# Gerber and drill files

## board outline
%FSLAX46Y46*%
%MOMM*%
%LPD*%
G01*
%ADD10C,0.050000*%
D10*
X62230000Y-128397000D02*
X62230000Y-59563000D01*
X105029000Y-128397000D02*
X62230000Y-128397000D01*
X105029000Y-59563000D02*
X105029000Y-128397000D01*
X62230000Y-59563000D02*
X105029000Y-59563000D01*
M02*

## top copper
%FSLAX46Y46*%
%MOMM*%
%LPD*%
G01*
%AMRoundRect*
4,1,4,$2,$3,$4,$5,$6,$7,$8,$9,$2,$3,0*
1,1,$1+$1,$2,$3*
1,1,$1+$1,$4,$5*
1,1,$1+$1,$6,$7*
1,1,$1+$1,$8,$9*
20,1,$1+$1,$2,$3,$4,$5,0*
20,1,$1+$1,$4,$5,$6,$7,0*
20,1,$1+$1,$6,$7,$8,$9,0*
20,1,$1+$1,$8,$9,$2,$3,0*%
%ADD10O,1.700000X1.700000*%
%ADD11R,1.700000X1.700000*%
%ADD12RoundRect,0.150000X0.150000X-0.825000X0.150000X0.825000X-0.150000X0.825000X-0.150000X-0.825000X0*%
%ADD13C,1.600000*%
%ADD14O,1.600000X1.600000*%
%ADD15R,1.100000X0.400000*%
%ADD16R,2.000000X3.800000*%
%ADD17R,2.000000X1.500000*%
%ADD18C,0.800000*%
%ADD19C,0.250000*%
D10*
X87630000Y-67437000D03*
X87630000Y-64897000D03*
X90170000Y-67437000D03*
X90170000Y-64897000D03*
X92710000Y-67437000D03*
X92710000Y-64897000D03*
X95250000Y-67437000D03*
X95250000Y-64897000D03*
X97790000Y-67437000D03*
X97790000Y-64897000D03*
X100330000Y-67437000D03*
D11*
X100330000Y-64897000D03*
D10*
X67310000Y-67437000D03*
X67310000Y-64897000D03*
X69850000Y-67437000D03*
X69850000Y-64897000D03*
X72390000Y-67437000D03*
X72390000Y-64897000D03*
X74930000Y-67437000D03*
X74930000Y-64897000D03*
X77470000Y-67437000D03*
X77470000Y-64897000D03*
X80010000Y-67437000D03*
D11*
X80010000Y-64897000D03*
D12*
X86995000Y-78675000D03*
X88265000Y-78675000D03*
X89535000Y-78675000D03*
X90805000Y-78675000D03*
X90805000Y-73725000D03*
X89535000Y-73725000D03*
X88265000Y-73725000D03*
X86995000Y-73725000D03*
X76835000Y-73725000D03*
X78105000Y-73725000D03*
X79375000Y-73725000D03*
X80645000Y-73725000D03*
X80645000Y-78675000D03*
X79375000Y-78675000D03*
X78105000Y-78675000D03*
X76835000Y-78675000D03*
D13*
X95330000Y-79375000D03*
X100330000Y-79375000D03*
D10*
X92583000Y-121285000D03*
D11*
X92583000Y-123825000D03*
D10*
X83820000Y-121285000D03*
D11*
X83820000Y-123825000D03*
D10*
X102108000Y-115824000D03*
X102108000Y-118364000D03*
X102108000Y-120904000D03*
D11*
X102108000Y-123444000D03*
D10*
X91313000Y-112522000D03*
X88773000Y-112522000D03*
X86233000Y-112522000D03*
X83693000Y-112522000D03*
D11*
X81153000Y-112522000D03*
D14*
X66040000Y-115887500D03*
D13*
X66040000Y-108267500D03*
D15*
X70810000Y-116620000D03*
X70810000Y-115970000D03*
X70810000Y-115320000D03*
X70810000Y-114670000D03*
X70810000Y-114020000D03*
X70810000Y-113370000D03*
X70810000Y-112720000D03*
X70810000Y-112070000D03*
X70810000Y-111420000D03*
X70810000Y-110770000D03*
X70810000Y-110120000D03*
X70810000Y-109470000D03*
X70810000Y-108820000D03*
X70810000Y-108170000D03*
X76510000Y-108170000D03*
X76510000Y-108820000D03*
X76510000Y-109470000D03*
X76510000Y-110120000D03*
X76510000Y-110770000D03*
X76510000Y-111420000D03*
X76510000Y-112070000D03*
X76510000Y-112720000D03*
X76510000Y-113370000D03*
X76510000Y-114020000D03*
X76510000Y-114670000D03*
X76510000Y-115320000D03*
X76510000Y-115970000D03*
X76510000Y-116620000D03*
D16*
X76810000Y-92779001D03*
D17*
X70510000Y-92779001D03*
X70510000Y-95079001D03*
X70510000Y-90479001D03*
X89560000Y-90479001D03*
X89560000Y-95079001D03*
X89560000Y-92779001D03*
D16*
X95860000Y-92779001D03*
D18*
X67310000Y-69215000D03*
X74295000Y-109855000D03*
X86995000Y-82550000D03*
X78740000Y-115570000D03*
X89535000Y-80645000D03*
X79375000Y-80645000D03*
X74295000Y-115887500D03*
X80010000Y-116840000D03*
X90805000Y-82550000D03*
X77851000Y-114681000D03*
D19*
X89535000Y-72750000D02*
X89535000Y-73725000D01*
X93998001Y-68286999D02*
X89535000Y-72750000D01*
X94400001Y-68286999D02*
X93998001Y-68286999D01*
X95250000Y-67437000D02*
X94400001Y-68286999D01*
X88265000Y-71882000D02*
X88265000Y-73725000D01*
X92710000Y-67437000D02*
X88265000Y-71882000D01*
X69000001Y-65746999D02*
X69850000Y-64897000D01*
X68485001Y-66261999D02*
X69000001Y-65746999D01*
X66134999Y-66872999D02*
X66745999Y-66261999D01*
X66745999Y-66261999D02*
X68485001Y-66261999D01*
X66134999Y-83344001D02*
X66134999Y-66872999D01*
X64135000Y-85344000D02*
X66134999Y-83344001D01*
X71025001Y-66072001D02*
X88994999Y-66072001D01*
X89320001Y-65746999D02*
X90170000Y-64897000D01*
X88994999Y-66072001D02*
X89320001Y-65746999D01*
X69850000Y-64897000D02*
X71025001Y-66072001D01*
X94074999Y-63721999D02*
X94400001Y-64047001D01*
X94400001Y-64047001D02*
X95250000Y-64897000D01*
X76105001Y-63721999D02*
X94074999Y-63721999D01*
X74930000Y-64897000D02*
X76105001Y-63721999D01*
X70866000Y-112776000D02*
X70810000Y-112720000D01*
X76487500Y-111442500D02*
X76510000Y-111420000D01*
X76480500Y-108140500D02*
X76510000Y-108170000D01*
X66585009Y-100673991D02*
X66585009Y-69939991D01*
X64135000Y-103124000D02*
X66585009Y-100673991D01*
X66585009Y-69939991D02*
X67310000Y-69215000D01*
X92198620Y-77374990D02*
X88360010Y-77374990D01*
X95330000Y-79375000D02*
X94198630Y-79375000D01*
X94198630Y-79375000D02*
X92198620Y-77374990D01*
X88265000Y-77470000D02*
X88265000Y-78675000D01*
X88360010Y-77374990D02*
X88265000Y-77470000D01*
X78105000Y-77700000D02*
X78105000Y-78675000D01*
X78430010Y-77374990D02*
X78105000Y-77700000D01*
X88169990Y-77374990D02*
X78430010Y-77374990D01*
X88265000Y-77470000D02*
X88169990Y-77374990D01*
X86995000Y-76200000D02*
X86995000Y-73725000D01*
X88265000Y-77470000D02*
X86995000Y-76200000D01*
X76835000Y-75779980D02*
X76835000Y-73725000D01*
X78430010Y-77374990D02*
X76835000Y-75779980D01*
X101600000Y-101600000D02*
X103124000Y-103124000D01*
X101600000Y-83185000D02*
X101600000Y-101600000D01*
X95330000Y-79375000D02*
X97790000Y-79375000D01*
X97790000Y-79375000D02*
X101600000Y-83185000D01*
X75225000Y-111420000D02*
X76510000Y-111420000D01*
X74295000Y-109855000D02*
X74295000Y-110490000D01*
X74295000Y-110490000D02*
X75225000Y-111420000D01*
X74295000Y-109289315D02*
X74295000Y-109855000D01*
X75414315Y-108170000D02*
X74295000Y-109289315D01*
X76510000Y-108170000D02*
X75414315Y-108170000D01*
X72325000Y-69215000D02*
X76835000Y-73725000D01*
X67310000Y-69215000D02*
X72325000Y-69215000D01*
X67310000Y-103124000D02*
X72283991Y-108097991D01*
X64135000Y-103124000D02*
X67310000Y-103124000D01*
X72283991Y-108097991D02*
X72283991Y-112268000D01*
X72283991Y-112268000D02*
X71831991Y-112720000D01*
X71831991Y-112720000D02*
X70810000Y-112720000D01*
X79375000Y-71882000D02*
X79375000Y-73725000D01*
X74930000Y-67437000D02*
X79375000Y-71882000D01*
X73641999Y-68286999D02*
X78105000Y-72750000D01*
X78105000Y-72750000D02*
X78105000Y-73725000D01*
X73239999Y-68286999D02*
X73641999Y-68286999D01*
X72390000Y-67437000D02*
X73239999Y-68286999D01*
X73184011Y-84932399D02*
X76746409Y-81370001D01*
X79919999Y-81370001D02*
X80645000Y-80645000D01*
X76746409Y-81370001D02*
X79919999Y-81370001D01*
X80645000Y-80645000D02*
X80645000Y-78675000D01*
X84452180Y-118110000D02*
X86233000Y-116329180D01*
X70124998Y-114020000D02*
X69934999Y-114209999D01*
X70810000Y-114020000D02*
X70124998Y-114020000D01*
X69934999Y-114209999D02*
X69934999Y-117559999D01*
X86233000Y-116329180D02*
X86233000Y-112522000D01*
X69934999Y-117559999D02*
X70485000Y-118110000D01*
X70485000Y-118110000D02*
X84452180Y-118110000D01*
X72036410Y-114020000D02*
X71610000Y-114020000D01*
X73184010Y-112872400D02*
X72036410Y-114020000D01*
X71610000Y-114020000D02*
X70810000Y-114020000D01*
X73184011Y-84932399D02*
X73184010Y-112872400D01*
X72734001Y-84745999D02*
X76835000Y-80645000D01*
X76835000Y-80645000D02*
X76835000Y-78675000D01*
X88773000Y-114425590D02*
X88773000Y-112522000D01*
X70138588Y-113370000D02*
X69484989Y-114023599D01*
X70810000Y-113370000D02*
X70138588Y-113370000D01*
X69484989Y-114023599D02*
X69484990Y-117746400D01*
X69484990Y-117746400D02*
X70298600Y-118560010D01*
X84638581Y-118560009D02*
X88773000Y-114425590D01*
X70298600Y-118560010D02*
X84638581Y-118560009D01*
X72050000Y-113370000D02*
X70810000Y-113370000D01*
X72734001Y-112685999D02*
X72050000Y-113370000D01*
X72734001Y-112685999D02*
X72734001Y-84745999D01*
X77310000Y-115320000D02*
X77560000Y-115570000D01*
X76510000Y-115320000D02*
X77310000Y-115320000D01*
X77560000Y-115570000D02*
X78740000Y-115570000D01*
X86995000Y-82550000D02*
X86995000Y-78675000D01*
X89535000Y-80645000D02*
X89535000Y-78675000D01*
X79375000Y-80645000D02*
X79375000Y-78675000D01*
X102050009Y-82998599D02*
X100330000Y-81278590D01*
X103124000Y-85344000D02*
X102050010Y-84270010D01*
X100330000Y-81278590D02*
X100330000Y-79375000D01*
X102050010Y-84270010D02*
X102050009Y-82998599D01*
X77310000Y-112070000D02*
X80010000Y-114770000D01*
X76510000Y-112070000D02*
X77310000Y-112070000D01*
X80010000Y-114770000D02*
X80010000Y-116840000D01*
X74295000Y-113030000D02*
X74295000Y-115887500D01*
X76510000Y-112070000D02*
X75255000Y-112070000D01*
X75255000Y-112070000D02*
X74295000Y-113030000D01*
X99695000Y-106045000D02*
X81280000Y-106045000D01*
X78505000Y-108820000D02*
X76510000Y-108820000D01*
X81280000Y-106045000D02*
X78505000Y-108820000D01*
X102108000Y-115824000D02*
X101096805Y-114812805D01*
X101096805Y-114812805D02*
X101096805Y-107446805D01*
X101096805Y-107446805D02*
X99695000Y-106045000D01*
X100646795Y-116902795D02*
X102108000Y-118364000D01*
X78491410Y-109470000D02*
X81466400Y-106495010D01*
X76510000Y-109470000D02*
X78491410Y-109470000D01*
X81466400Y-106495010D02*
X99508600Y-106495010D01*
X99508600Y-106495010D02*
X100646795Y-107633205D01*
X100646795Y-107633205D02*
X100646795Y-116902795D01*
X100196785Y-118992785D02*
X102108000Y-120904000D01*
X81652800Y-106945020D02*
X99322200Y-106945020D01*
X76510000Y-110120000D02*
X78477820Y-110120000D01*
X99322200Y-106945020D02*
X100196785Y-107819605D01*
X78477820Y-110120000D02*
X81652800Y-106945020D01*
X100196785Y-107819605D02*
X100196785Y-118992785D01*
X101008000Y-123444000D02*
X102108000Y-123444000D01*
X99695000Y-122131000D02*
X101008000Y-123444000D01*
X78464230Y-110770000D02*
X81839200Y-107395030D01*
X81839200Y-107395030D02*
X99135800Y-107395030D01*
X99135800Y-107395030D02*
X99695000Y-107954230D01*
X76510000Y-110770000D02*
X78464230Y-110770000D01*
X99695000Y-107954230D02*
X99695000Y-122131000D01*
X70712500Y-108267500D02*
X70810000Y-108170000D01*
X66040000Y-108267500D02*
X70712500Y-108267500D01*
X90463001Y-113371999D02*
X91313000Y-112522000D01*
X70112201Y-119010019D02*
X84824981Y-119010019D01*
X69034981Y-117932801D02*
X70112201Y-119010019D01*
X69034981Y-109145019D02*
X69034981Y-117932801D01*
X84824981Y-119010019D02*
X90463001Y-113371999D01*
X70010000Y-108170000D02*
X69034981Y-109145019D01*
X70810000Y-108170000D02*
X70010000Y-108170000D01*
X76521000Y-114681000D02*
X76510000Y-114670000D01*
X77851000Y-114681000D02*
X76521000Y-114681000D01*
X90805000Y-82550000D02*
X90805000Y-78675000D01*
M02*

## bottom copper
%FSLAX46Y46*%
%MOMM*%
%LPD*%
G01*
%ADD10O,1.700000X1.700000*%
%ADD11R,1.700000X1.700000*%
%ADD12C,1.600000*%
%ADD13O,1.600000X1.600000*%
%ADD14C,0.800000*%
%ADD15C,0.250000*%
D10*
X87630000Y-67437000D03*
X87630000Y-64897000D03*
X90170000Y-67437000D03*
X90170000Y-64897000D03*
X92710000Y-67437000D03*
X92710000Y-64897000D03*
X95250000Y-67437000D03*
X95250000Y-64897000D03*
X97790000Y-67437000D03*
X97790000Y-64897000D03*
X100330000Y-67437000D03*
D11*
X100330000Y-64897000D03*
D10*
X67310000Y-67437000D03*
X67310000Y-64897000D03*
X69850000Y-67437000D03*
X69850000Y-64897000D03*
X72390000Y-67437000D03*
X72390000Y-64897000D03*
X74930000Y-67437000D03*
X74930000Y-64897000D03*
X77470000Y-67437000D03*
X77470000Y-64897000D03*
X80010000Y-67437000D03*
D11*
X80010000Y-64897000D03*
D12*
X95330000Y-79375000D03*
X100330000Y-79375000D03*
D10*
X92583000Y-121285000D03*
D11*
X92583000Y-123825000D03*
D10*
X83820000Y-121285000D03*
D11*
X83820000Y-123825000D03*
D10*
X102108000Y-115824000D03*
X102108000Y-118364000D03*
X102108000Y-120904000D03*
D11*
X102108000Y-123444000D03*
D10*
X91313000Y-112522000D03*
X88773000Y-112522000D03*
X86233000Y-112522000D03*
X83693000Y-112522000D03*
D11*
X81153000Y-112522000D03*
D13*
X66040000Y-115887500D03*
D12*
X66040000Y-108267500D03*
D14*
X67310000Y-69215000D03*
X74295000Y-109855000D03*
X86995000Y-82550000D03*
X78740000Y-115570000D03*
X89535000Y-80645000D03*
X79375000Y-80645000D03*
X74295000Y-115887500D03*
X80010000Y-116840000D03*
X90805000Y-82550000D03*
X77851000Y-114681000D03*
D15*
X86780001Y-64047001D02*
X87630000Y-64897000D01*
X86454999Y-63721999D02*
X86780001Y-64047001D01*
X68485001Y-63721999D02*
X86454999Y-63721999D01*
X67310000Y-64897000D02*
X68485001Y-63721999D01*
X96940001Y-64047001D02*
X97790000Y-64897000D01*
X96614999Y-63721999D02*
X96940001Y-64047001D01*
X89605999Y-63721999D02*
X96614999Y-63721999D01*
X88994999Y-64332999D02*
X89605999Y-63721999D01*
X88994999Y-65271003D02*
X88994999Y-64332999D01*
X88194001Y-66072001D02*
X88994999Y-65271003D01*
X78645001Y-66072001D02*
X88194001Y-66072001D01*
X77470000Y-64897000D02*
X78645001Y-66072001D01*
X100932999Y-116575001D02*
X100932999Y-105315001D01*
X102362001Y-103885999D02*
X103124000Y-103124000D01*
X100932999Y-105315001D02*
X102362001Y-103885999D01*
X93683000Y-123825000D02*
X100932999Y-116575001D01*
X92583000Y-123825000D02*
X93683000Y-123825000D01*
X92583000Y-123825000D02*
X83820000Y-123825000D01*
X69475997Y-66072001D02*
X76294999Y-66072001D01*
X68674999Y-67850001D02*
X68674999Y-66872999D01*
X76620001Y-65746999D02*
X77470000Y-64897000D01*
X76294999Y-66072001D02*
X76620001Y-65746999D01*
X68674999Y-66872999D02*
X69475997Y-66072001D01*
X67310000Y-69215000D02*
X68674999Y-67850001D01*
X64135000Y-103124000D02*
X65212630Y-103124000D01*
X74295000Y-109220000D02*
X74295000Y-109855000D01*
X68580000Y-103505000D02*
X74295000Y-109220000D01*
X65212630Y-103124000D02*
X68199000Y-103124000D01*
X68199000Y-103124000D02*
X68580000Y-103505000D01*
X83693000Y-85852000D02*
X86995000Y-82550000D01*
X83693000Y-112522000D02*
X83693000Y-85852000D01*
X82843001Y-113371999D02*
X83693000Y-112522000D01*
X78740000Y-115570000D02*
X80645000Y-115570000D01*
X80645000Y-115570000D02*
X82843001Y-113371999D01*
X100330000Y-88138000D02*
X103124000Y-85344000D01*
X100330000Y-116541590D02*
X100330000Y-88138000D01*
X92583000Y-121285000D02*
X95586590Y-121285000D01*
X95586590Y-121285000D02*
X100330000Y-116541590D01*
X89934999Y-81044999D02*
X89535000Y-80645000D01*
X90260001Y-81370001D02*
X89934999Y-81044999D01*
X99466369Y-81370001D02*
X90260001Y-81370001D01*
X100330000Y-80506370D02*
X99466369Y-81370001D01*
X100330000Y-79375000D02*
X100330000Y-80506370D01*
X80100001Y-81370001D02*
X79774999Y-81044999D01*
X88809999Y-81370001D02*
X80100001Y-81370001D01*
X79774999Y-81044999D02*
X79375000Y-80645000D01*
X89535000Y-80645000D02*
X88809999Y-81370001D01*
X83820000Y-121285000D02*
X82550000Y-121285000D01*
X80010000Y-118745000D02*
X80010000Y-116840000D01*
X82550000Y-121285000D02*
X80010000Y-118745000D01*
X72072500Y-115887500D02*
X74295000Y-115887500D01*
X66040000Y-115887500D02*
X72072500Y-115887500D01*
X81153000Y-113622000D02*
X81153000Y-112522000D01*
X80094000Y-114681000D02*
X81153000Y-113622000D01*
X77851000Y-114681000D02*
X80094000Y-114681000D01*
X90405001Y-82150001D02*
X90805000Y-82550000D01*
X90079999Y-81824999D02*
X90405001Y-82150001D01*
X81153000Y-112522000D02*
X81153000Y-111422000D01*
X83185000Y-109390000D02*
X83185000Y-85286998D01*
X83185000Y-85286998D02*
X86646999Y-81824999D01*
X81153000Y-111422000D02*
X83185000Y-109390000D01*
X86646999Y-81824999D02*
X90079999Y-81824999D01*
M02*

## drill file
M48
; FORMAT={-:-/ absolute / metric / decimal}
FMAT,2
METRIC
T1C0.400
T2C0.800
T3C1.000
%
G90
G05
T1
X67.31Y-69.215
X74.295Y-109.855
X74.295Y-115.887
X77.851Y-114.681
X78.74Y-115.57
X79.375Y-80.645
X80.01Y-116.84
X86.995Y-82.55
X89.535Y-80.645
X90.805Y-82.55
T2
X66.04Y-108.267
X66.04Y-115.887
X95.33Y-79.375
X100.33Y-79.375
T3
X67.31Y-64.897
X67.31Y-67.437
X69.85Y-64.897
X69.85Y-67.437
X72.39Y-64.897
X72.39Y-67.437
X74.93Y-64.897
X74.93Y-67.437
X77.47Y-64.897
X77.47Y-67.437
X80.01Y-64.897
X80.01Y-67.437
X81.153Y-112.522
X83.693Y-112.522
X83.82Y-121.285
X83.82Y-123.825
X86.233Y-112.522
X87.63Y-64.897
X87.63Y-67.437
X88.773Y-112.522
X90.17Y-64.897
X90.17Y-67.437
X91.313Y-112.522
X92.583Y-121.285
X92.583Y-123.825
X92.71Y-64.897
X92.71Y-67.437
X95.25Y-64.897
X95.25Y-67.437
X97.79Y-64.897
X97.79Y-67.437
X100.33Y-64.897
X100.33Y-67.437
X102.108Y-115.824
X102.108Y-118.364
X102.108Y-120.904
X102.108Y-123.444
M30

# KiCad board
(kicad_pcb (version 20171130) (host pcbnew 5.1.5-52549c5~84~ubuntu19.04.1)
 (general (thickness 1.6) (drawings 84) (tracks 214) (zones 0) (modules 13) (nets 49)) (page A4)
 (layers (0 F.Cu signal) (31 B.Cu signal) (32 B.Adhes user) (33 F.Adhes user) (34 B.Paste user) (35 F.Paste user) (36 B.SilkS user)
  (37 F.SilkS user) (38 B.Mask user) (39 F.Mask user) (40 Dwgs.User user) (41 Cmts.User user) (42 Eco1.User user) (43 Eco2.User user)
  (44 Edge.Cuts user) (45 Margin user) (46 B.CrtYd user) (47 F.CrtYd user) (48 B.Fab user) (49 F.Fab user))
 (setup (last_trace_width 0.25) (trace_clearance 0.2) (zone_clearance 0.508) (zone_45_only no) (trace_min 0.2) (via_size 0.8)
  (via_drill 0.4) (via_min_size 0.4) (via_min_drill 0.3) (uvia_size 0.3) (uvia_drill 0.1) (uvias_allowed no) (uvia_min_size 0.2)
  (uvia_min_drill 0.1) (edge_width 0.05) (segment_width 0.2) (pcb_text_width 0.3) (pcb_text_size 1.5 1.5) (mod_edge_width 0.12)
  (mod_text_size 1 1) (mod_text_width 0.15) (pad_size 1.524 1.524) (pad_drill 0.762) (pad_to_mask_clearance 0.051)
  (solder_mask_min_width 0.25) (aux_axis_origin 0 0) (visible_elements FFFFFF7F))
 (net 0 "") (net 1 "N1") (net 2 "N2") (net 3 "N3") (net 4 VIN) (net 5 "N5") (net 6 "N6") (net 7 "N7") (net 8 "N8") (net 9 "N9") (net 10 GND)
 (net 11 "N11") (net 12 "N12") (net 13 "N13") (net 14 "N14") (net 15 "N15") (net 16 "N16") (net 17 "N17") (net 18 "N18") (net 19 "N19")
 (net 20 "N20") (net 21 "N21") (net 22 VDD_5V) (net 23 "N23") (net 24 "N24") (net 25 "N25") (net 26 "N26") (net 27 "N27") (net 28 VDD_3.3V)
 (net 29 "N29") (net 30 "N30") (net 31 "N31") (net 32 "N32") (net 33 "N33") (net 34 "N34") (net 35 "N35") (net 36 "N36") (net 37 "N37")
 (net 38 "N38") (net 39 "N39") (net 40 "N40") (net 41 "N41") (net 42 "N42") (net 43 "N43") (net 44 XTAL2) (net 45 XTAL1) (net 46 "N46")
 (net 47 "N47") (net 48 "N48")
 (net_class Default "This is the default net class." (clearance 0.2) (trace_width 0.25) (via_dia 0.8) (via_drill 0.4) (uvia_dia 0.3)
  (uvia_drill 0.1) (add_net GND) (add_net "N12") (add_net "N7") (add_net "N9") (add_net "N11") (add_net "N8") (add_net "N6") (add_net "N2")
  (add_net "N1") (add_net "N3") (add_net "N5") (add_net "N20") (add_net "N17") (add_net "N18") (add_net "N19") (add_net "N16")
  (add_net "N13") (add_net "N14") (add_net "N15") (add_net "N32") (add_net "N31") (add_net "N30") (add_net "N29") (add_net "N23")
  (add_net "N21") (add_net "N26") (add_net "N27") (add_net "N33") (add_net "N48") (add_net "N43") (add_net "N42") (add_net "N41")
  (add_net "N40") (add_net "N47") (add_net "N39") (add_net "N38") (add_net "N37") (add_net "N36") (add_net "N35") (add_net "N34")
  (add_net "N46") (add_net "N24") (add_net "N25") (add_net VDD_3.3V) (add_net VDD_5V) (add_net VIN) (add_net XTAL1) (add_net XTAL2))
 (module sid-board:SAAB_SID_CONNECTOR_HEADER (layer F.Cu) (at 93.98 66.04)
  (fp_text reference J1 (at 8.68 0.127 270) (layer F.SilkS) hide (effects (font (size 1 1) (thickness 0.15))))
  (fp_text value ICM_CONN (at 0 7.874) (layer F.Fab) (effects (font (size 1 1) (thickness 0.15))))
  (pad 7 thru_hole oval (at -6.35 1.397 270) (size 1.7 1.7) (drill 1) (layers *.Cu *.Mask) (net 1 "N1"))
  (pad 6 thru_hole oval (at -6.35 -1.143 270) (size 1.7 1.7) (drill 1) (layers *.Cu *.Mask) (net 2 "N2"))
  (pad 8 thru_hole oval (at -3.81 1.397 270) (size 1.7 1.7) (drill 1) (layers *.Cu *.Mask) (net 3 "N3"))
  (pad 5 thru_hole oval (at -3.81 -1.143 270) (size 1.7 1.7) (drill 1) (layers *.Cu *.Mask) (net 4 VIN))
  (pad 9 thru_hole oval (at -1.27 1.397 270) (size 1.7 1.7) (drill 1) (layers *.Cu *.Mask) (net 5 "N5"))
  (pad 4 thru_hole oval (at -1.27 -1.143 270) (size 1.7 1.7) (drill 1) (layers *.Cu *.Mask) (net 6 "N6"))
  (pad 10 thru_hole oval (at 1.27 1.397 270) (size 1.7 1.7) (drill 1) (layers *.Cu *.Mask) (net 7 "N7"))
  (pad 3 thru_hole oval (at 1.27 -1.143 270) (size 1.7 1.7) (drill 1) (layers *.Cu *.Mask) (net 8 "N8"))
  (pad 11 thru_hole oval (at 3.81 1.397 270) (size 1.7 1.7) (drill 1) (layers *.Cu *.Mask) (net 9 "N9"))
  (pad 2 thru_hole oval (at 3.81 -1.143 270) (size 1.7 1.7) (drill 1) (layers *.Cu *.Mask) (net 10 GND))
  (pad 12 thru_hole oval (at 6.35 1.397 270) (size 1.7 1.7) (drill 1) (layers *.Cu *.Mask) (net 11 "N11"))
  (pad 1 thru_hole rect (at 6.35 -1.143 270) (size 1.7 1.7) (drill 1) (layers *.Cu *.Mask) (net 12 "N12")))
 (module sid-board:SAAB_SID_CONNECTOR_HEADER (layer F.Cu) (at 73.66 66.04)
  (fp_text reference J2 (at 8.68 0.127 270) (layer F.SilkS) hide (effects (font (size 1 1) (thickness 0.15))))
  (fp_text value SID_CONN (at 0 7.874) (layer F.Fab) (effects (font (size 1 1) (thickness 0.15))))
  (pad 7 thru_hole oval (at -6.35 1.397 270) (size 1.7 1.7) (drill 1) (layers *.Cu *.Mask) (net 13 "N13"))
  (pad 6 thru_hole oval (at -6.35 -1.143 270) (size 1.7 1.7) (drill 1) (layers *.Cu *.Mask) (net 2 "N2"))
  (pad 8 thru_hole oval (at -3.81 1.397 270) (size 1.7 1.7) (drill 1) (layers *.Cu *.Mask) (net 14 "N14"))
  (pad 5 thru_hole oval (at -3.81 -1.143 270) (size 1.7 1.7) (drill 1) (layers *.Cu *.Mask) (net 4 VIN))
  (pad 9 thru_hole oval (at -1.27 1.397 270) (size 1.7 1.7) (drill 1) (layers *.Cu *.Mask) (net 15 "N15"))
  (pad 4 thru_hole oval (at -1.27 -1.143 270) (size 1.7 1.7) (drill 1) (layers *.Cu *.Mask) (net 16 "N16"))
  (pad 10 thru_hole oval (at 1.27 1.397 270) (size 1.7 1.7) (drill 1) (layers *.Cu *.Mask) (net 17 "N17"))
  (pad 3 thru_hole oval (at 1.27 -1.143 270) (size 1.7 1.7) (drill 1) (layers *.Cu *.Mask) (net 8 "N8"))
  (pad 11 thru_hole oval (at 3.81 1.397 270) (size 1.7 1.7) (drill 1) (layers *.Cu *.Mask) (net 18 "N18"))
  (pad 2 thru_hole oval (at 3.81 -1.143 270) (size 1.7 1.7) (drill 1) (layers *.Cu *.Mask) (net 10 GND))
  (pad 12 thru_hole oval (at 6.35 1.397 270) (size 1.7 1.7) (drill 1) (layers *.Cu *.Mask) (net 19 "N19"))
  (pad 1 thru_hole rect (at 6.35 -1.143 270) (size 1.7 1.7) (drill 1) (layers *.Cu *.Mask) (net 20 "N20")))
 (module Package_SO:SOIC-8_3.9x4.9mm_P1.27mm (layer F.Cu) (at 88.9 76.2 90)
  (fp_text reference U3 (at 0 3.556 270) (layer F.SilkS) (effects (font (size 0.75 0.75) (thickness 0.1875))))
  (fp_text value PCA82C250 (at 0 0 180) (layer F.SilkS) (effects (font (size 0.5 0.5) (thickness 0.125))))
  (pad 1 smd roundrect (at -2.475 -1.905 90) (size 1.95 0.6) (layers F.Cu F.Paste F.Mask) (roundrect_rratio 0.25) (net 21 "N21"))
  (pad 2 smd roundrect (at -2.475 -0.635 90) (size 1.95 0.6) (layers F.Cu F.Paste F.Mask) (roundrect_rratio 0.25) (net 10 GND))
  (pad 3 smd roundrect (at -2.475 0.635 90) (size 1.95 0.6) (layers F.Cu F.Paste F.Mask) (roundrect_rratio 0.25) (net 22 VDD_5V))
  (pad 4 smd roundrect (at -2.475 1.905 90) (size 1.95 0.6) (layers F.Cu F.Paste F.Mask) (roundrect_rratio 0.25) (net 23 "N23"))
  (pad 5 smd roundrect (at 2.475 1.905 90) (size 1.95 0.6) (layers F.Cu F.Paste F.Mask) (roundrect_rratio 0.25) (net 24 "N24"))
  (pad 6 smd roundrect (at 2.475 0.635 90) (size 1.95 0.6) (layers F.Cu F.Paste F.Mask) (roundrect_rratio 0.25) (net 7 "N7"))
  (pad 7 smd roundrect (at 2.475 -0.635 90) (size 1.95 0.6) (layers F.Cu F.Paste F.Mask) (roundrect_rratio 0.25) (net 5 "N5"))
  (pad 8 smd roundrect (at 2.475 -1.905 90) (size 1.95 0.6) (layers F.Cu F.Paste F.Mask) (roundrect_rratio 0.25) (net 10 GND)))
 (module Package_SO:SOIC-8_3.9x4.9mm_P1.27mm (layer F.Cu) (at 78.74 76.2 90)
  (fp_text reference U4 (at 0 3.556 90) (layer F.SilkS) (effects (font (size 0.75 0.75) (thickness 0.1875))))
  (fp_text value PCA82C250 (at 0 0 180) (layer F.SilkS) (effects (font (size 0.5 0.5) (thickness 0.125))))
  (pad 8 smd roundrect (at 2.475 -1.905 90) (size 1.95 0.6) (layers F.Cu F.Paste F.Mask) (roundrect_rratio 0.25) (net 10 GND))
  (pad 7 smd roundrect (at 2.475 -0.635 90) (size 1.95 0.6) (layers F.Cu F.Paste F.Mask) (roundrect_rratio 0.25) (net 15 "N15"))
  (pad 6 smd roundrect (at 2.475 0.635 90) (size 1.95 0.6) (layers F.Cu F.Paste F.Mask) (roundrect_rratio 0.25) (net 17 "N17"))
  (pad 5 smd roundrect (at 2.475 1.905 90) (size 1.95 0.6) (layers F.Cu F.Paste F.Mask) (roundrect_rratio 0.25) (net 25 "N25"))
  (pad 4 smd roundrect (at -2.475 1.905 90) (size 1.95 0.6) (layers F.Cu F.Paste F.Mask) (roundrect_rratio 0.25) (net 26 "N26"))
  (pad 3 smd roundrect (at -2.475 0.635 90) (size 1.95 0.6) (layers F.Cu F.Paste F.Mask) (roundrect_rratio 0.25) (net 22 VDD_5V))
  (pad 2 smd roundrect (at -2.475 -0.635 90) (size 1.95 0.6) (layers F.Cu F.Paste F.Mask) (roundrect_rratio 0.25) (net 10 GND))
  (pad 1 smd roundrect (at -2.475 -1.905 90) (size 1.95 0.6) (layers F.Cu F.Paste F.Mask) (roundrect_rratio 0.25) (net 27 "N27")))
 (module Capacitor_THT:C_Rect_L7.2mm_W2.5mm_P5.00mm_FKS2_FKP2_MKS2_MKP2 (layer F.Cu) (at 100.33 79.375 180)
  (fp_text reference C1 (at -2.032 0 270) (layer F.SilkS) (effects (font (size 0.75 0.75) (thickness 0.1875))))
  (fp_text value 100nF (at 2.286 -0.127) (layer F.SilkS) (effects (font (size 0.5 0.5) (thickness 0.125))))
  (pad 2 thru_hole circle (at 5 0 180) (size 1.6 1.6) (drill 0.8) (layers *.Cu *.Mask) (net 10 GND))
  (pad 1 thru_hole circle (at 0 0 180) (size 1.6 1.6) (drill 0.8) (layers *.Cu *.Mask) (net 22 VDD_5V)))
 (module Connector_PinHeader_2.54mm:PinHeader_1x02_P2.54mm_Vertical (layer F.Cu) (at 92.583 123.825 180)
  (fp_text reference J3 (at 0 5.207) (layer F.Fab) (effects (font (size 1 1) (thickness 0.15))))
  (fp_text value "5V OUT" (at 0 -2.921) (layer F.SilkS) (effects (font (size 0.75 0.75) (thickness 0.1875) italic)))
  (pad 2 thru_hole oval (at 0 2.54 180) (size 1.7 1.7) (drill 1) (layers *.Cu *.Mask) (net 22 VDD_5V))
  (pad 1 thru_hole rect (at 0 0 180) (size 1.7 1.7) (drill 1) (layers *.Cu *.Mask) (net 10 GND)))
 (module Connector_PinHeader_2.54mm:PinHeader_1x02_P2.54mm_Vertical (layer F.Cu) (at 83.82 123.825 180)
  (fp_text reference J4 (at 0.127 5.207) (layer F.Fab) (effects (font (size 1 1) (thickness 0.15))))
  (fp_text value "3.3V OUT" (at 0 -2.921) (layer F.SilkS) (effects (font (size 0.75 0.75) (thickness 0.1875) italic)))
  (pad 2 thru_hole oval (at 0 2.54 180) (size 1.7 1.7) (drill 1) (layers *.Cu *.Mask) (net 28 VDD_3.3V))
  (pad 1 thru_hole rect (at 0 0 180) (size 1.7 1.7) (drill 1) (layers *.Cu *.Mask) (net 10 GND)))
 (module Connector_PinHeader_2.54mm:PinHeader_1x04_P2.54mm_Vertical (layer F.Cu) (at 102.108 123.444 180)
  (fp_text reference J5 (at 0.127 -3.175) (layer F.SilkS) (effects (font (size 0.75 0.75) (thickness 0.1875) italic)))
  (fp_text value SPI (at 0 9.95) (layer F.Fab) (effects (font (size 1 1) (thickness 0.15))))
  (pad 4 thru_hole oval (at 0 7.62 180) (size 1.7 1.7) (drill 1) (layers *.Cu *.Mask) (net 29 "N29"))
  (pad 3 thru_hole oval (at 0 5.08 180) (size 1.7 1.7) (drill 1) (layers *.Cu *.Mask) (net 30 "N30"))
  (pad 2 thru_hole oval (at 0 2.54 180) (size 1.7 1.7) (drill 1) (layers *.Cu *.Mask) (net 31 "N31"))
  (pad 1 thru_hole rect (at 0 0 180) (size 1.7 1.7) (drill 1) (layers *.Cu *.Mask) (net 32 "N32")))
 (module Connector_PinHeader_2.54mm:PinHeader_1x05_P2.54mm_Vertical (layer F.Cu) (at 81.153 112.522 90)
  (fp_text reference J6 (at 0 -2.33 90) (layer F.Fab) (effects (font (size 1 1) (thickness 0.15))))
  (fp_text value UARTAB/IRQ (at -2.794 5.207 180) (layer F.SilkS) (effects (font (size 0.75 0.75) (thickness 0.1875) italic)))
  (pad 5 thru_hole oval (at 0 10.16 90) (size 1.7 1.7) (drill 1) (layers *.Cu *.Mask) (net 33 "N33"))
  (pad 4 thru_hole oval (at 0 7.62 90) (size 1.7 1.7) (drill 1) (layers *.Cu *.Mask) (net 27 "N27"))
  (pad 3 thru_hole oval (at 0 5.08 90) (size 1.7 1.7) (drill 1) (layers *.Cu *.Mask) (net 26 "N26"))
  (pad 2 thru_hole oval (at 0 2.54 90) (size 1.7 1.7) (drill 1) (layers *.Cu *.Mask) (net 21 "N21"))
  (pad 1 thru_hole rect (at 0 0 90) (size 1.7 1.7) (drill 1) (layers *.Cu *.Mask) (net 23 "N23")))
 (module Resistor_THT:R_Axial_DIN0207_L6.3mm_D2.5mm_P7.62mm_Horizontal (layer F.Cu) (at 66.04 108.2675 270)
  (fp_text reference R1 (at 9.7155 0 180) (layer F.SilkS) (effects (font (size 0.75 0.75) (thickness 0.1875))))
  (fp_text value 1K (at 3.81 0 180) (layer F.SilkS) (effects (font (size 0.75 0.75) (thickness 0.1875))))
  (pad 2 thru_hole oval (at 7.62 0 270) (size 1.6 1.6) (drill 0.8) (layers *.Cu *.Mask) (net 28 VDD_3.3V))
  (pad 1 thru_hole circle (at 0 0 270) (size 1.6 1.6) (drill 0.8) (layers *.Cu *.Mask) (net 33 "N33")))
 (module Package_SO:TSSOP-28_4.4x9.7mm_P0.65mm (layer F.Cu) (at 73.66 112.395 180)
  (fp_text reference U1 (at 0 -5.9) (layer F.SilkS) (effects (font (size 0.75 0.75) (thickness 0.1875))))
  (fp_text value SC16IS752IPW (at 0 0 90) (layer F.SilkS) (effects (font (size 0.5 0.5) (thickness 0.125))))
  (pad 28 smd rect (at 2.85 -4.225 180) (size 1.1 0.4) (layers F.Cu F.Paste F.Mask) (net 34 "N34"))
  (pad 27 smd rect (at 2.85 -3.575 180) (size 1.1 0.4) (layers F.Cu F.Paste F.Mask) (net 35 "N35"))
  (pad 26 smd rect (at 2.85 -2.925 180) (size 1.1 0.4) (layers F.Cu F.Paste F.Mask) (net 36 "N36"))
  (pad 25 smd rect (at 2.85 -2.275 180) (size 1.1 0.4) (layers F.Cu F.Paste F.Mask) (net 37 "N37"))
  (pad 24 smd rect (at 2.85 -1.625 180) (size 1.1 0.4) (layers F.Cu F.Paste F.Mask) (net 26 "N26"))
  (pad 23 smd rect (at 2.85 -0.975 180) (size 1.1 0.4) (layers F.Cu F.Paste F.Mask) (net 27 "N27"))
  (pad 22 smd rect (at 2.85 -0.325 180) (size 1.1 0.4) (layers F.Cu F.Paste F.Mask) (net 10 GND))
  (pad 21 smd rect (at 2.85 0.325 180) (size 1.1 0.4) (layers F.Cu F.Paste F.Mask) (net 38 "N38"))
  (pad 20 smd rect (at 2.85 0.975 180) (size 1.1 0.4) (layers F.Cu F.Paste F.Mask) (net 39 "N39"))
  (pad 19 smd rect (at 2.85 1.625 180) (size 1.1 0.4) (layers F.Cu F.Paste F.Mask) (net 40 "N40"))
  (pad 18 smd rect (at 2.85 2.275 180) (size 1.1 0.4) (layers F.Cu F.Paste F.Mask) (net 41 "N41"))
  (pad 17 smd rect (at 2.85 2.925 180) (size 1.1 0.4) (layers F.Cu F.Paste F.Mask) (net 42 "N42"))
  (pad 16 smd rect (at 2.85 3.575 180) (size 1.1 0.4) (layers F.Cu F.Paste F.Mask) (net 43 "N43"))
  (pad 15 smd rect (at 2.85 4.225 180) (size 1.1 0.4) (layers F.Cu F.Paste F.Mask) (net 33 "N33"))
  (pad 14 smd rect (at -2.85 4.225 180) (size 1.1 0.4) (layers F.Cu F.Paste F.Mask) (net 10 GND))
  (pad 13 smd rect (at -2.85 3.575 180) (size 1.1 0.4) (layers F.Cu F.Paste F.Mask) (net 29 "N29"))
  (pad 12 smd rect (at -2.85 2.925 180) (size 1.1 0.4) (layers F.Cu F.Paste F.Mask) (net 30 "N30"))
  (pad 11 smd rect (at -2.85 2.275 180) (size 1.1 0.4) (layers F.Cu F.Paste F.Mask) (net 31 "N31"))
  (pad 10 smd rect (at -2.85 1.625 180) (size 1.1 0.4) (layers F.Cu F.Paste F.Mask) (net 32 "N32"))
  (pad 9 smd rect (at -2.85 0.975 180) (size 1.1 0.4) (layers F.Cu F.Paste F.Mask) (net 10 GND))
  (pad 8 smd rect (at -2.85 0.325 180) (size 1.1 0.4) (layers F.Cu F.Paste F.Mask) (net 28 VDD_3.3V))
  (pad 7 smd rect (at -2.85 -0.325 180) (size 1.1 0.4) (layers F.Cu F.Paste F.Mask) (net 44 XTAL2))
  (pad 6 smd rect (at -2.85 -0.975 180) (size 1.1 0.4) (layers F.Cu F.Paste F.Mask) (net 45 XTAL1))
  (pad 5 smd rect (at -2.85 -1.625 180) (size 1.1 0.4) (layers F.Cu F.Paste F.Mask) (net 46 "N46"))
  (pad 4 smd rect (at -2.85 -2.275 180) (size 1.1 0.4) (layers F.Cu F.Paste F.Mask) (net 23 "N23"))
  (pad 3 smd rect (at -2.85 -2.925 180) (size 1.1 0.4) (layers F.Cu F.Paste F.Mask) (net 21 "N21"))
  (pad 2 smd rect (at -2.85 -3.575 180) (size 1.1 0.4) (layers F.Cu F.Paste F.Mask) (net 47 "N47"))
  (pad 1 smd rect (at -2.85 -4.225 180) (size 1.1 0.4) (layers F.Cu F.Paste F.Mask) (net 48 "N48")))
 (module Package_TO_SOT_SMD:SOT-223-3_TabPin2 (layer F.Cu) (at 73.66 92.779001)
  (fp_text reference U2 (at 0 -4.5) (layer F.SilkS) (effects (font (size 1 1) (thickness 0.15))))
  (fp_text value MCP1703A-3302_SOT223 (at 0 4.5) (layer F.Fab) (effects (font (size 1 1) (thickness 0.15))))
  (pad 2 smd rect (at 3.15 0) (size 2 3.8) (layers F.Cu F.Paste F.Mask) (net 10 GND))
  (pad 2 smd rect (at -3.15 0) (size 2 1.5) (layers F.Cu F.Paste F.Mask) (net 10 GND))
  (pad 3 smd rect (at -3.15 2.3) (size 2 1.5) (layers F.Cu F.Paste F.Mask) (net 28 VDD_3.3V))
  (pad 1 smd rect (at -3.15 -2.3) (size 2 1.5) (layers F.Cu F.Paste F.Mask) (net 4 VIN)))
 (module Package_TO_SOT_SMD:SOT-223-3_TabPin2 (layer F.Cu) (at 92.71 92.779001)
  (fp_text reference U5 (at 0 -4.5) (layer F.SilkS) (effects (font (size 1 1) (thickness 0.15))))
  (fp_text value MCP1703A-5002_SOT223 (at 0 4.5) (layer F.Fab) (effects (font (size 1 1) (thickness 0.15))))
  (pad 1 smd rect (at -3.15 -2.3) (size 2 1.5) (layers F.Cu F.Paste F.Mask) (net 4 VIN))
  (pad 3 smd rect (at -3.15 2.3) (size 2 1.5) (layers F.Cu F.Paste F.Mask) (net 22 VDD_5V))
  (pad 2 smd rect (at -3.15 0) (size 2 1.5) (layers F.Cu F.Paste F.Mask) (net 10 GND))
  (pad 2 smd rect (at 3.15 0) (size 2 3.8) (layers F.Cu F.Paste F.Mask) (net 10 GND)))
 (gr_line (start 62.23 128.397) (end 62.23 59.563) (layer Edge.Cuts) (width 0.05))
 (gr_line (start 105.029 128.397) (end 62.23 128.397) (layer Edge.Cuts) (width 0.05))
 (gr_line (start 105.029 59.563) (end 105.029 128.397) (layer Edge.Cuts) (width 0.05))
 (gr_line (start 62.23 59.563) (end 105.029 59.563) (layer Edge.Cuts) (width 0.05))
 (segment (start 89.535 72.75) (end 89.535 73.725) (width 0.25) (layer F.Cu) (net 7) (status 30))
 (segment (start 93.998001 68.286999) (end 89.535 72.75) (width 0.25) (layer F.Cu) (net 7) (status 20))
 (segment (start 94.400001 68.286999) (end 93.998001 68.286999) (width 0.25) (layer F.Cu) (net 7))
 (segment (start 95.25 67.437) (end 94.400001 68.286999) (width 0.25) (layer F.Cu) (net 7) (status 10))
 (segment (start 88.265 71.882) (end 88.265 73.725) (width 0.25) (layer F.Cu) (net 5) (status 20))
 (segment (start 92.71 67.437) (end 88.265 71.882) (width 0.25) (layer F.Cu) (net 5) (status 10))
 (segment (start 86.780001 64.047001) (end 87.63 64.897) (width 0.25) (layer B.Cu) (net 2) (status 20))
 (segment (start 86.454999 63.721999) (end 86.780001 64.047001) (width 0.25) (layer B.Cu) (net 2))
 (segment (start 68.485001 63.721999) (end 86.454999 63.721999) (width 0.25) (layer B.Cu) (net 2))
 (segment (start 67.31 64.897) (end 68.485001 63.721999) (width 0.25) (layer B.Cu) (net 2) (status 10))
 (segment (start 69.000001 65.746999) (end 69.85 64.897) (width 0.25) (layer F.Cu) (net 4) (status 20))
 (segment (start 68.485001 66.261999) (end 69.000001 65.746999) (width 0.25) (layer F.Cu) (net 4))
 (segment (start 66.134999 66.872999) (end 66.745999 66.261999) (width 0.25) (layer F.Cu) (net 4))
 (segment (start 66.745999 66.261999) (end 68.485001 66.261999) (width 0.25) (layer F.Cu) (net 4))
 (segment (start 66.134999 83.344001) (end 66.134999 66.872999) (width 0.25) (layer F.Cu) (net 4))
 (segment (start 64.135 85.344) (end 66.134999 83.344001) (width 0.25) (layer F.Cu) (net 4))
 (segment (start 71.025001 66.072001) (end 88.994999 66.072001) (width 0.25) (layer F.Cu) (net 4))
 (segment (start 89.320001 65.746999) (end 90.17 64.897) (width 0.25) (layer F.Cu) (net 4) (status 20))
 (segment (start 88.994999 66.072001) (end 89.320001 65.746999) (width 0.25) (layer F.Cu) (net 4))
 (segment (start 69.85 64.897) (end 71.025001 66.072001) (width 0.25) (layer F.Cu) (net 4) (status 10))
 (segment (start 94.074999 63.721999) (end 94.400001 64.047001) (width 0.25) (layer F.Cu) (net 8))
 (segment (start 94.400001 64.047001) (end 95.25 64.897) (width 0.25) (layer F.Cu) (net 8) (status 20))
 (segment (start 76.105001 63.721999) (end 94.074999 63.721999) (width 0.25) (layer F.Cu) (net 8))
 (segment (start 74.93 64.897) (end 76.105001 63.721999) (width 0.25) (layer F.Cu) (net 8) (status 10))
 (via (at 67.31 69.215) (size 0.8) (drill 0.4) (layers F.Cu B.Cu) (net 10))
 (via (at 74.295 109.855) (size 0.8) (drill 0.4) (layers F.Cu B.Cu) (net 10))
 (segment (start 96.940001 64.047001) (end 97.79 64.897) (width 0.25) (layer B.Cu) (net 10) (status 20))
 (segment (start 96.614999 63.721999) (end 96.940001 64.047001) (width 0.25) (layer B.Cu) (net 10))
 (segment (start 89.605999 63.721999) (end 96.614999 63.721999) (width 0.25) (layer B.Cu) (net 10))
 (segment (start 88.994999 64.332999) (end 89.605999 63.721999) (width 0.25) (layer B.Cu) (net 10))
 (segment (start 88.994999 65.271003) (end 88.994999 64.332999) (width 0.25) (layer B.Cu) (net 10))
 (segment (start 88.194001 66.072001) (end 88.994999 65.271003) (width 0.25) (layer B.Cu) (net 10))
 (segment (start 78.645001 66.072001) (end 88.194001 66.072001) (width 0.25) (layer B.Cu) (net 10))
 (segment (start 77.47 64.897) (end 78.645001 66.072001) (width 0.25) (layer B.Cu) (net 10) (status 10))
 (segment (start 70.866 112.776) (end 70.81 112.72) (width 0.25) (layer F.Cu) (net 10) (status 30))
 (segment (start 76.4875 111.4425) (end 76.51 111.42) (width 0.25) (layer F.Cu) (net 10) (status 30))
 (segment (start 76.4805 108.1405) (end 76.51 108.17) (width 0.25) (layer F.Cu) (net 10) (status 30))
 (segment (start 100.932999 116.575001) (end 100.932999 105.315001) (width 0.25) (layer B.Cu) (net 10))
 (segment (start 102.362001 103.885999) (end 103.124 103.124) (width 0.25) (layer B.Cu) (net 10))
 (segment (start 100.932999 105.315001) (end 102.362001 103.885999) (width 0.25) (layer B.Cu) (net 10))
 (segment (start 93.683 123.825) (end 100.932999 116.575001) (width 0.25) (layer B.Cu) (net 10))
 (segment (start 92.583 123.825) (end 93.683 123.825) (width 0.25) (layer B.Cu) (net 10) (status 10))
 (segment (start 92.583 123.825) (end 83.82 123.825) (width 0.25) (layer B.Cu) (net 10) (status 30))
 (segment (start 66.585009 100.673991) (end 66.585009 69.939991) (width 0.25) (layer F.Cu) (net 10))
 (segment (start 64.135 103.124) (end 66.585009 100.673991) (width 0.25) (layer F.Cu) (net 10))
 (segment (start 66.585009 69.939991) (end 67.31 69.215) (width 0.25) (layer F.Cu) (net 10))
 (segment (start 69.475997 66.072001) (end 76.294999 66.072001) (width 0.25) (layer B.Cu) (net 10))
 (segment (start 68.674999 67.850001) (end 68.674999 66.872999) (width 0.25) (layer B.Cu) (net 10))
 (segment (start 76.620001 65.746999) (end 77.47 64.897) (width 0.25) (layer B.Cu) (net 10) (status 20))
 (segment (start 76.294999 66.072001) (end 76.620001 65.746999) (width 0.25) (layer B.Cu) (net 10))
 (segment (start 68.674999 66.872999) (end 69.475997 66.072001) (width 0.25) (layer B.Cu) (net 10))
 (segment (start 67.31 69.215) (end 68.674999 67.850001) (width 0.25) (layer B.Cu) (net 10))
 (segment (start 92.19862 77.37499) (end 88.36001 77.37499) (width 0.25) (layer F.Cu) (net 10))
 (segment (start 95.33 79.375) (end 94.19863 79.375) (width 0.25) (layer F.Cu) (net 10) (status 10))
 (segment (start 94.19863 79.375) (end 92.19862 77.37499) (width 0.25) (layer F.Cu) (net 10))
 (segment (start 88.265 77.47) (end 88.265 78.675) (width 0.25) (layer F.Cu) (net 10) (status 20))
 (segment (start 88.36001 77.37499) (end 88.265 77.47) (width 0.25) (layer F.Cu) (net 10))
 (segment (start 78.105 77.7) (end 78.105 78.675) (width 0.25) (layer F.Cu) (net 10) (status 30))
 (segment (start 78.43001 77.37499) (end 78.105 77.7) (width 0.25) (layer F.Cu) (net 10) (status 20))
 (segment (start 88.16999 77.37499) (end 78.43001 77.37499) (width 0.25) (layer F.Cu) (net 10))
 (segment (start 88.265 77.47) (end 88.16999 77.37499) (width 0.25) (layer F.Cu) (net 10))
 (segment (start 86.995 76.2) (end 86.995 73.725) (width 0.25) (layer F.Cu) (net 10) (status 20))
 (segment (start 88.265 77.47) (end 86.995 76.2) (width 0.25) (layer F.Cu) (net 10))
 (segment (start 76.835 75.77998) (end 76.835 73.725) (width 0.25) (layer F.Cu) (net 10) (status 20))
 (segment (start 78.43001 77.37499) (end 76.835 75.77998) (width 0.25) (layer F.Cu) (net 10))
 (segment (start 101.6 101.6) (end 103.124 103.124) (width 0.25) (layer F.Cu) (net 10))
 (segment (start 101.6 83.185) (end 101.6 101.6) (width 0.25) (layer F.Cu) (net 10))
 (segment (start 95.33 79.375) (end 97.79 79.375) (width 0.25) (layer F.Cu) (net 10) (status 10))
 (segment (start 97.79 79.375) (end 101.6 83.185) (width 0.25) (layer F.Cu) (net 10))
 (segment (start 75.225 111.42) (end 76.51 111.42) (width 0.25) (layer F.Cu) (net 10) (status 20))
 (segment (start 74.295 109.855) (end 74.295 110.49) (width 0.25) (layer F.Cu) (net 10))
 (segment (start 74.295 110.49) (end 75.225 111.42) (width 0.25) (layer F.Cu) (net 10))
 (segment (start 74.295 109.289315) (end 74.295 109.855) (width 0.25) (layer F.Cu) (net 10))
 (segment (start 75.414315 108.17) (end 74.295 109.289315) (width 0.25) (layer F.Cu) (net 10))
 (segment (start 76.51 108.17) (end 75.414315 108.17) (width 0.25) (layer F.Cu) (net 10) (status 10))
 (segment (start 64.135 103.124) (end 65.21263 103.124) (width 0.25) (layer B.Cu) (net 10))
 (segment (start 74.295 109.22) (end 74.295 109.855) (width 0.25) (layer B.Cu) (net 10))
 (segment (start 68.58 103.505) (end 74.295 109.22) (width 0.25) (layer B.Cu) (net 10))
 (segment (start 65.21263 103.124) (end 68.199 103.124) (width 0.25) (layer B.Cu) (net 10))
 (segment (start 68.199 103.124) (end 68.58 103.505) (width 0.25) (layer B.Cu) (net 10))
 (segment (start 72.325 69.215) (end 76.835 73.725) (width 0.25) (layer F.Cu) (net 10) (status 20))
 (segment (start 67.31 69.215) (end 72.325 69.215) (width 0.25) (layer F.Cu) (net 10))
 (segment (start 67.31 103.124) (end 72.283991 108.097991) (width 0.25) (layer F.Cu) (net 10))
 (segment (start 64.135 103.124) (end 67.31 103.124) (width 0.25) (layer F.Cu) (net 10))
 (segment (start 72.283991 108.097991) (end 72.283991 112.268) (width 0.25) (layer F.Cu) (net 10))
 (segment (start 72.283991 112.268) (end 71.831991 112.72) (width 0.25) (layer F.Cu) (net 10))
 (segment (start 71.831991 112.72) (end 70.81 112.72) (width 0.25) (layer F.Cu) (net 10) (status 20))
 (segment (start 79.375 71.882) (end 79.375 73.725) (width 0.25) (layer F.Cu) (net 17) (status 20))
 (segment (start 74.93 67.437) (end 79.375 71.882) (width 0.25) (layer F.Cu) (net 17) (status 10))
 (segment (start 73.641999 68.286999) (end 78.105 72.75) (width 0.25) (layer F.Cu) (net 15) (status 20))
 (segment (start 78.105 72.75) (end 78.105 73.725) (width 0.25) (layer F.Cu) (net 15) (status 30))
 (segment (start 73.239999 68.286999) (end 73.641999 68.286999) (width 0.25) (layer F.Cu) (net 15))
 (segment (start 72.39 67.437) (end 73.239999 68.286999) (width 0.25) (layer F.Cu) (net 15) (status 10))
 (segment (start 73.184011 84.932399) (end 76.746409 81.370001) (width 0.25) (layer F.Cu) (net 26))
 (segment (start 79.919999 81.370001) (end 80.645 80.645) (width 0.25) (layer F.Cu) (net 26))
 (segment (start 76.746409 81.370001) (end 79.919999 81.370001) (width 0.25) (layer F.Cu) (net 26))
 (segment (start 80.645 80.645) (end 80.645 78.675) (width 0.25) (layer F.Cu) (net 26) (status 20))
 (segment (start 84.45218 118.11) (end 86.233 116.32918) (width 0.25) (layer F.Cu) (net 26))
 (segment (start 70.124998 114.02) (end 69.934999 114.209999) (width 0.25) (layer F.Cu) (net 26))
 (segment (start 70.81 114.02) (end 70.124998 114.02) (width 0.25) (layer F.Cu) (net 26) (status 10))
 (segment (start 69.934999 114.209999) (end 69.934999 117.559999) (width 0.25) (layer F.Cu) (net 26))
 (segment (start 86.233 116.32918) (end 86.233 112.522) (width 0.25) (layer F.Cu) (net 26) (status 20))
 (segment (start 69.934999 117.559999) (end 70.485 118.11) (width 0.25) (layer F.Cu) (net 26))
 (segment (start 70.485 118.11) (end 84.45218 118.11) (width 0.25) (layer F.Cu) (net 26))
 (segment (start 72.03641 114.02) (end 71.61 114.02) (width 0.25) (layer F.Cu) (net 26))
 (segment (start 73.18401 112.8724) (end 72.03641 114.02) (width 0.25) (layer F.Cu) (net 26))
 (segment (start 71.61 114.02) (end 70.81 114.02) (width 0.25) (layer F.Cu) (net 26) (status 20))
 (segment (start 73.184011 84.932399) (end 73.18401 112.8724) (width 0.25) (layer F.Cu) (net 26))
 (segment (start 72.734001 84.745999) (end 76.835 80.645) (width 0.25) (layer F.Cu) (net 27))
 (segment (start 76.835 80.645) (end 76.835 78.675) (width 0.25) (layer F.Cu) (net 27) (status 20))
 (segment (start 88.773 114.42559) (end 88.773 112.522) (width 0.25) (layer F.Cu) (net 27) (status 20))
 (segment (start 70.138588 113.37) (end 69.484989 114.023599) (width 0.25) (layer F.Cu) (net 27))
 (segment (start 70.81 113.37) (end 70.138588 113.37) (width 0.25) (layer F.Cu) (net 27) (status 10))
 (segment (start 69.484989 114.023599) (end 69.48499 117.7464) (width 0.25) (layer F.Cu) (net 27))
 (segment (start 69.48499 117.7464) (end 70.2986 118.56001) (width 0.25) (layer F.Cu) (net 27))
 (segment (start 84.638581 118.560009) (end 88.773 114.42559) (width 0.25) (layer F.Cu) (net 27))
 (segment (start 70.2986 118.56001) (end 84.638581 118.560009) (width 0.25) (layer F.Cu) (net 27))
 (segment (start 72.05 113.37) (end 70.81 113.37) (width 0.25) (layer F.Cu) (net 27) (status 20))
 (segment (start 72.734001 112.685999) (end 72.05 113.37) (width 0.25) (layer F.Cu) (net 27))
 (segment (start 72.734001 112.685999) (end 72.734001 84.745999) (width 0.25) (layer F.Cu) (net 27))
 (via (at 86.995 82.55) (size 0.8) (drill 0.4) (layers F.Cu B.Cu) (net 21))
 (segment (start 77.31 115.32) (end 77.56 115.57) (width 0.25) (layer F.Cu) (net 21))
 (segment (start 76.51 115.32) (end 77.31 115.32) (width 0.25) (layer F.Cu) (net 21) (status 10))
 (segment (start 77.56 115.57) (end 78.74 115.57) (width 0.25) (layer F.Cu) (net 21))
 (via (at 78.74 115.57) (size 0.8) (drill 0.4) (layers F.Cu B.Cu) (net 21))
 (segment (start 86.995 82.55) (end 86.995 78.675) (width 0.25) (layer F.Cu) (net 21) (status 20))
 (segment (start 83.693 85.852) (end 86.995 82.55) (width 0.25) (layer B.Cu) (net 21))
 (segment (start 83.693 112.522) (end 83.693 85.852) (width 0.25) (layer B.Cu) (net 21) (status 10))
 (segment (start 82.843001 113.371999) (end 83.693 112.522) (width 0.25) (layer B.Cu) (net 21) (status 20))
 (segment (start 78.74 115.57) (end 80.645 115.57) (width 0.25) (layer B.Cu) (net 21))
 (segment (start 80.645 115.57) (end 82.843001 113.371999) (width 0.25) (layer B.Cu) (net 21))
 (via (at 89.535 80.645) (size 0.8) (drill 0.4) (layers F.Cu B.Cu) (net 22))
 (via (at 79.375 80.645) (size 0.8) (drill 0.4) (layers F.Cu B.Cu) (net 22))
 (segment (start 100.33 88.138) (end 103.124 85.344) (width 0.25) (layer B.Cu) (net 22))
 (segment (start 100.33 116.54159) (end 100.33 88.138) (width 0.25) (layer B.Cu) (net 22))
 (segment (start 92.583 121.285) (end 95.58659 121.285) (width 0.25) (layer B.Cu) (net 22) (status 10))
 (segment (start 95.58659 121.285) (end 100.33 116.54159) (width 0.25) (layer B.Cu) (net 22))
 (segment (start 89.934999 81.044999) (end 89.535 80.645) (width 0.25) (layer B.Cu) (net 22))
 (segment (start 90.260001 81.370001) (end 89.934999 81.044999) (width 0.25) (layer B.Cu) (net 22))
 (segment (start 99.466369 81.370001) (end 90.260001 81.370001) (width 0.25) (layer B.Cu) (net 22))
 (segment (start 100.33 80.50637) (end 99.466369 81.370001) (width 0.25) (layer B.Cu) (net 22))
 (segment (start 100.33 79.375) (end 100.33 80.50637) (width 0.25) (layer B.Cu) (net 22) (status 10))
 (segment (start 80.100001 81.370001) (end 79.774999 81.044999) (width 0.25) (layer B.Cu) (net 22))
 (segment (start 88.809999 81.370001) (end 80.100001 81.370001) (width 0.25) (layer B.Cu) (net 22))
 (segment (start 79.774999 81.044999) (end 79.375 80.645) (width 0.25) (layer B.Cu) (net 22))
 (segment (start 89.535 80.645) (end 88.809999 81.370001) (width 0.25) (layer B.Cu) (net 22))
 (segment (start 89.535 80.645) (end 89.535 78.675) (width 0.25) (layer F.Cu) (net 22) (status 20))
 (segment (start 79.375 80.645) (end 79.375 78.675) (width 0.25) (layer F.Cu) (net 22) (status 20))
 (segment (start 102.050009 82.998599) (end 100.33 81.27859) (width 0.25) (layer F.Cu) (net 22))
 (segment (start 103.124 85.344) (end 102.05001 84.27001) (width 0.25) (layer F.Cu) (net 22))
 (segment (start 100.33 81.27859) (end 100.33 79.375) (width 0.25) (layer F.Cu) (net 22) (status 20))
 (segment (start 102.05001 84.27001) (end 102.050009 82.998599) (width 0.25) (layer F.Cu) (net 22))
 (via (at 74.295 115.8875) (size 0.8) (drill 0.4) (layers F.Cu B.Cu) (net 28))
 (segment (start 77.31 112.07) (end 80.01 114.77) (width 0.25) (layer F.Cu) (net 28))
 (segment (start 76.51 112.07) (end 77.31 112.07) (width 0.25) (layer F.Cu) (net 28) (status 10))
 (segment (start 80.01 114.77) (end 80.01 116.84) (width 0.25) (layer F.Cu) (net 28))
 (via (at 80.01 116.84) (size 0.8) (drill 0.4) (layers F.Cu B.Cu) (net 28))
 (segment (start 83.82 121.285) (end 82.55 121.285) (width 0.25) (layer B.Cu) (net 28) (status 10))
 (segment (start 80.01 118.745) (end 80.01 116.84) (width 0.25) (layer B.Cu) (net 28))
 (segment (start 82.55 121.285) (end 80.01 118.745) (width 0.25) (layer B.Cu) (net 28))
 (segment (start 72.0725 115.8875) (end 74.295 115.8875) (width 0.25) (layer B.Cu) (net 28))
 (segment (start 66.04 115.8875) (end 72.0725 115.8875) (width 0.25) (layer B.Cu) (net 28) (status 10))
 (segment (start 74.295 113.03) (end 74.295 115.8875) (width 0.25) (layer F.Cu) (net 28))
 (segment (start 76.51 112.07) (end 75.255 112.07) (width 0.25) (layer F.Cu) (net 28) (status 10))
 (segment (start 75.255 112.07) (end 74.295 113.03) (width 0.25) (layer F.Cu) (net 28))
 (segment (start 99.695 106.045) (end 81.28 106.045) (width 0.25) (layer F.Cu) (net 29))
 (segment (start 78.505 108.82) (end 76.51 108.82) (width 0.25) (layer F.Cu) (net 29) (status 20))
 (segment (start 81.28 106.045) (end 78.505 108.82) (width 0.25) (layer F.Cu) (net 29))
 (segment (start 102.108 115.824) (end 101.096805 114.812805) (width 0.25) (layer F.Cu) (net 29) (status 10))
 (segment (start 101.096805 114.812805) (end 101.096805 107.446805) (width 0.25) (layer F.Cu) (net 29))
 (segment (start 101.096805 107.446805) (end 99.695 106.045) (width 0.25) (layer F.Cu) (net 29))
 (segment (start 100.646795 116.902795) (end 102.108 118.364) (width 0.25) (layer F.Cu) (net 30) (status 20))
 (segment (start 78.49141 109.47) (end 81.4664 106.49501) (width 0.25) (layer F.Cu) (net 30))
 (segment (start 76.51 109.47) (end 78.49141 109.47) (width 0.25) (layer F.Cu) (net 30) (status 10))
 (segment (start 81.4664 106.49501) (end 99.5086 106.49501) (width 0.25) (layer F.Cu) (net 30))
 (segment (start 99.5086 106.49501) (end 100.646795 107.633205) (width 0.25) (layer F.Cu) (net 30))
 (segment (start 100.646795 107.633205) (end 100.646795 116.902795) (width 0.25) (layer F.Cu) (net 30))
 (segment (start 100.196785 118.992785) (end 102.108 120.904) (width 0.25) (layer F.Cu) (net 31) (status 20))
 (segment (start 81.6528 106.94502) (end 99.3222 106.94502) (width 0.25) (layer F.Cu) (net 31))
 (segment (start 76.51 110.12) (end 78.47782 110.12) (width 0.25) (layer F.Cu) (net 31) (status 10))
 (segment (start 99.3222 106.94502) (end 100.196785 107.819605) (width 0.25) (layer F.Cu) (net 31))
 (segment (start 78.47782 110.12) (end 81.6528 106.94502) (width 0.25) (layer F.Cu) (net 31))
 (segment (start 100.196785 107.819605) (end 100.196785 118.992785) (width 0.25) (layer F.Cu) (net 31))
 (segment (start 101.008 123.444) (end 102.108 123.444) (width 0.25) (layer F.Cu) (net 32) (status 20))
 (segment (start 99.695 122.131) (end 101.008 123.444) (width 0.25) (layer F.Cu) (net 32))
 (segment (start 78.46423 110.77) (end 81.8392 107.39503) (width 0.25) (layer F.Cu) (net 32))
 (segment (start 81.8392 107.39503) (end 99.1358 107.39503) (width 0.25) (layer F.Cu) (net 32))
 (segment (start 99.1358 107.39503) (end 99.695 107.95423) (width 0.25) (layer F.Cu) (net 32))
 (segment (start 76.51 110.77) (end 78.46423 110.77) (width 0.25) (layer F.Cu) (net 32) (status 10))
 (segment (start 99.695 107.95423) (end 99.695 122.131) (width 0.25) (layer F.Cu) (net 32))
 (segment (start 70.7125 108.2675) (end 70.81 108.17) (width 0.25) (layer F.Cu) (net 33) (status 30))
 (segment (start 66.04 108.2675) (end 70.7125 108.2675) (width 0.25) (layer F.Cu) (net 33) (status 30))
 (segment (start 90.463001 113.371999) (end 91.313 112.522) (width 0.25) (layer F.Cu) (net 33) (status 20))
 (segment (start 70.112201 119.010019) (end 84.824981 119.010019) (width 0.25) (layer F.Cu) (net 33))
 (segment (start 69.034981 117.932801) (end 70.112201 119.010019) (width 0.25) (layer F.Cu) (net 33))
 (segment (start 69.034981 109.145019) (end 69.034981 117.932801) (width 0.25) (layer F.Cu) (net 33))
 (segment (start 84.824981 119.010019) (end 90.463001 113.371999) (width 0.25) (layer F.Cu) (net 33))
 (segment (start 70.01 108.17) (end 69.034981 109.145019) (width 0.25) (layer F.Cu) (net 33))
 (segment (start 70.81 108.17) (end 70.01 108.17) (width 0.25) (layer F.Cu) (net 33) (status 10))
 (via (at 90.805 82.55) (size 0.8) (drill 0.4) (layers F.Cu B.Cu) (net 23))
 (via (at 77.851 114.681) (size 0.8) (drill 0.4) (layers F.Cu B.Cu) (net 23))
 (segment (start 76.521 114.681) (end 76.51 114.67) (width 0.25) (layer F.Cu) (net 23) (status 30))
 (segment (start 77.851 114.681) (end 76.521 114.681) (width 0.25) (layer F.Cu) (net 23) (status 20))
 (segment (start 81.153 113.622) (end 81.153 112.522) (width 0.25) (layer B.Cu) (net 23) (status 20))
 (segment (start 80.094 114.681) (end 81.153 113.622) (width 0.25) (layer B.Cu) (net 23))
 (segment (start 77.851 114.681) (end 80.094 114.681) (width 0.25) (layer B.Cu) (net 23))
 (segment (start 90.805 82.55) (end 90.805 78.675) (width 0.25) (layer F.Cu) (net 23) (status 20))
 (segment (start 90.405001 82.150001) (end 90.805 82.55) (width 0.25) (layer B.Cu) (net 23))
 (segment (start 90.079999 81.824999) (end 90.405001 82.150001) (width 0.25) (layer B.Cu) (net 23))
 (segment (start 81.153 112.522) (end 81.153 111.422) (width 0.25) (layer B.Cu) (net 23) (status 10))
 (segment (start 83.185 109.39) (end 83.185 85.286998) (width 0.25) (layer B.Cu) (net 23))
 (segment (start 83.185 85.286998) (end 86.646999 81.824999) (width 0.25) (layer B.Cu) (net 23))
 (segment (start 81.153 111.422) (end 83.185 109.39) (width 0.25) (layer B.Cu) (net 23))
 (segment (start 86.646999 81.824999) (end 90.079999 81.824999) (width 0.25) (layer B.Cu) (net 23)))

